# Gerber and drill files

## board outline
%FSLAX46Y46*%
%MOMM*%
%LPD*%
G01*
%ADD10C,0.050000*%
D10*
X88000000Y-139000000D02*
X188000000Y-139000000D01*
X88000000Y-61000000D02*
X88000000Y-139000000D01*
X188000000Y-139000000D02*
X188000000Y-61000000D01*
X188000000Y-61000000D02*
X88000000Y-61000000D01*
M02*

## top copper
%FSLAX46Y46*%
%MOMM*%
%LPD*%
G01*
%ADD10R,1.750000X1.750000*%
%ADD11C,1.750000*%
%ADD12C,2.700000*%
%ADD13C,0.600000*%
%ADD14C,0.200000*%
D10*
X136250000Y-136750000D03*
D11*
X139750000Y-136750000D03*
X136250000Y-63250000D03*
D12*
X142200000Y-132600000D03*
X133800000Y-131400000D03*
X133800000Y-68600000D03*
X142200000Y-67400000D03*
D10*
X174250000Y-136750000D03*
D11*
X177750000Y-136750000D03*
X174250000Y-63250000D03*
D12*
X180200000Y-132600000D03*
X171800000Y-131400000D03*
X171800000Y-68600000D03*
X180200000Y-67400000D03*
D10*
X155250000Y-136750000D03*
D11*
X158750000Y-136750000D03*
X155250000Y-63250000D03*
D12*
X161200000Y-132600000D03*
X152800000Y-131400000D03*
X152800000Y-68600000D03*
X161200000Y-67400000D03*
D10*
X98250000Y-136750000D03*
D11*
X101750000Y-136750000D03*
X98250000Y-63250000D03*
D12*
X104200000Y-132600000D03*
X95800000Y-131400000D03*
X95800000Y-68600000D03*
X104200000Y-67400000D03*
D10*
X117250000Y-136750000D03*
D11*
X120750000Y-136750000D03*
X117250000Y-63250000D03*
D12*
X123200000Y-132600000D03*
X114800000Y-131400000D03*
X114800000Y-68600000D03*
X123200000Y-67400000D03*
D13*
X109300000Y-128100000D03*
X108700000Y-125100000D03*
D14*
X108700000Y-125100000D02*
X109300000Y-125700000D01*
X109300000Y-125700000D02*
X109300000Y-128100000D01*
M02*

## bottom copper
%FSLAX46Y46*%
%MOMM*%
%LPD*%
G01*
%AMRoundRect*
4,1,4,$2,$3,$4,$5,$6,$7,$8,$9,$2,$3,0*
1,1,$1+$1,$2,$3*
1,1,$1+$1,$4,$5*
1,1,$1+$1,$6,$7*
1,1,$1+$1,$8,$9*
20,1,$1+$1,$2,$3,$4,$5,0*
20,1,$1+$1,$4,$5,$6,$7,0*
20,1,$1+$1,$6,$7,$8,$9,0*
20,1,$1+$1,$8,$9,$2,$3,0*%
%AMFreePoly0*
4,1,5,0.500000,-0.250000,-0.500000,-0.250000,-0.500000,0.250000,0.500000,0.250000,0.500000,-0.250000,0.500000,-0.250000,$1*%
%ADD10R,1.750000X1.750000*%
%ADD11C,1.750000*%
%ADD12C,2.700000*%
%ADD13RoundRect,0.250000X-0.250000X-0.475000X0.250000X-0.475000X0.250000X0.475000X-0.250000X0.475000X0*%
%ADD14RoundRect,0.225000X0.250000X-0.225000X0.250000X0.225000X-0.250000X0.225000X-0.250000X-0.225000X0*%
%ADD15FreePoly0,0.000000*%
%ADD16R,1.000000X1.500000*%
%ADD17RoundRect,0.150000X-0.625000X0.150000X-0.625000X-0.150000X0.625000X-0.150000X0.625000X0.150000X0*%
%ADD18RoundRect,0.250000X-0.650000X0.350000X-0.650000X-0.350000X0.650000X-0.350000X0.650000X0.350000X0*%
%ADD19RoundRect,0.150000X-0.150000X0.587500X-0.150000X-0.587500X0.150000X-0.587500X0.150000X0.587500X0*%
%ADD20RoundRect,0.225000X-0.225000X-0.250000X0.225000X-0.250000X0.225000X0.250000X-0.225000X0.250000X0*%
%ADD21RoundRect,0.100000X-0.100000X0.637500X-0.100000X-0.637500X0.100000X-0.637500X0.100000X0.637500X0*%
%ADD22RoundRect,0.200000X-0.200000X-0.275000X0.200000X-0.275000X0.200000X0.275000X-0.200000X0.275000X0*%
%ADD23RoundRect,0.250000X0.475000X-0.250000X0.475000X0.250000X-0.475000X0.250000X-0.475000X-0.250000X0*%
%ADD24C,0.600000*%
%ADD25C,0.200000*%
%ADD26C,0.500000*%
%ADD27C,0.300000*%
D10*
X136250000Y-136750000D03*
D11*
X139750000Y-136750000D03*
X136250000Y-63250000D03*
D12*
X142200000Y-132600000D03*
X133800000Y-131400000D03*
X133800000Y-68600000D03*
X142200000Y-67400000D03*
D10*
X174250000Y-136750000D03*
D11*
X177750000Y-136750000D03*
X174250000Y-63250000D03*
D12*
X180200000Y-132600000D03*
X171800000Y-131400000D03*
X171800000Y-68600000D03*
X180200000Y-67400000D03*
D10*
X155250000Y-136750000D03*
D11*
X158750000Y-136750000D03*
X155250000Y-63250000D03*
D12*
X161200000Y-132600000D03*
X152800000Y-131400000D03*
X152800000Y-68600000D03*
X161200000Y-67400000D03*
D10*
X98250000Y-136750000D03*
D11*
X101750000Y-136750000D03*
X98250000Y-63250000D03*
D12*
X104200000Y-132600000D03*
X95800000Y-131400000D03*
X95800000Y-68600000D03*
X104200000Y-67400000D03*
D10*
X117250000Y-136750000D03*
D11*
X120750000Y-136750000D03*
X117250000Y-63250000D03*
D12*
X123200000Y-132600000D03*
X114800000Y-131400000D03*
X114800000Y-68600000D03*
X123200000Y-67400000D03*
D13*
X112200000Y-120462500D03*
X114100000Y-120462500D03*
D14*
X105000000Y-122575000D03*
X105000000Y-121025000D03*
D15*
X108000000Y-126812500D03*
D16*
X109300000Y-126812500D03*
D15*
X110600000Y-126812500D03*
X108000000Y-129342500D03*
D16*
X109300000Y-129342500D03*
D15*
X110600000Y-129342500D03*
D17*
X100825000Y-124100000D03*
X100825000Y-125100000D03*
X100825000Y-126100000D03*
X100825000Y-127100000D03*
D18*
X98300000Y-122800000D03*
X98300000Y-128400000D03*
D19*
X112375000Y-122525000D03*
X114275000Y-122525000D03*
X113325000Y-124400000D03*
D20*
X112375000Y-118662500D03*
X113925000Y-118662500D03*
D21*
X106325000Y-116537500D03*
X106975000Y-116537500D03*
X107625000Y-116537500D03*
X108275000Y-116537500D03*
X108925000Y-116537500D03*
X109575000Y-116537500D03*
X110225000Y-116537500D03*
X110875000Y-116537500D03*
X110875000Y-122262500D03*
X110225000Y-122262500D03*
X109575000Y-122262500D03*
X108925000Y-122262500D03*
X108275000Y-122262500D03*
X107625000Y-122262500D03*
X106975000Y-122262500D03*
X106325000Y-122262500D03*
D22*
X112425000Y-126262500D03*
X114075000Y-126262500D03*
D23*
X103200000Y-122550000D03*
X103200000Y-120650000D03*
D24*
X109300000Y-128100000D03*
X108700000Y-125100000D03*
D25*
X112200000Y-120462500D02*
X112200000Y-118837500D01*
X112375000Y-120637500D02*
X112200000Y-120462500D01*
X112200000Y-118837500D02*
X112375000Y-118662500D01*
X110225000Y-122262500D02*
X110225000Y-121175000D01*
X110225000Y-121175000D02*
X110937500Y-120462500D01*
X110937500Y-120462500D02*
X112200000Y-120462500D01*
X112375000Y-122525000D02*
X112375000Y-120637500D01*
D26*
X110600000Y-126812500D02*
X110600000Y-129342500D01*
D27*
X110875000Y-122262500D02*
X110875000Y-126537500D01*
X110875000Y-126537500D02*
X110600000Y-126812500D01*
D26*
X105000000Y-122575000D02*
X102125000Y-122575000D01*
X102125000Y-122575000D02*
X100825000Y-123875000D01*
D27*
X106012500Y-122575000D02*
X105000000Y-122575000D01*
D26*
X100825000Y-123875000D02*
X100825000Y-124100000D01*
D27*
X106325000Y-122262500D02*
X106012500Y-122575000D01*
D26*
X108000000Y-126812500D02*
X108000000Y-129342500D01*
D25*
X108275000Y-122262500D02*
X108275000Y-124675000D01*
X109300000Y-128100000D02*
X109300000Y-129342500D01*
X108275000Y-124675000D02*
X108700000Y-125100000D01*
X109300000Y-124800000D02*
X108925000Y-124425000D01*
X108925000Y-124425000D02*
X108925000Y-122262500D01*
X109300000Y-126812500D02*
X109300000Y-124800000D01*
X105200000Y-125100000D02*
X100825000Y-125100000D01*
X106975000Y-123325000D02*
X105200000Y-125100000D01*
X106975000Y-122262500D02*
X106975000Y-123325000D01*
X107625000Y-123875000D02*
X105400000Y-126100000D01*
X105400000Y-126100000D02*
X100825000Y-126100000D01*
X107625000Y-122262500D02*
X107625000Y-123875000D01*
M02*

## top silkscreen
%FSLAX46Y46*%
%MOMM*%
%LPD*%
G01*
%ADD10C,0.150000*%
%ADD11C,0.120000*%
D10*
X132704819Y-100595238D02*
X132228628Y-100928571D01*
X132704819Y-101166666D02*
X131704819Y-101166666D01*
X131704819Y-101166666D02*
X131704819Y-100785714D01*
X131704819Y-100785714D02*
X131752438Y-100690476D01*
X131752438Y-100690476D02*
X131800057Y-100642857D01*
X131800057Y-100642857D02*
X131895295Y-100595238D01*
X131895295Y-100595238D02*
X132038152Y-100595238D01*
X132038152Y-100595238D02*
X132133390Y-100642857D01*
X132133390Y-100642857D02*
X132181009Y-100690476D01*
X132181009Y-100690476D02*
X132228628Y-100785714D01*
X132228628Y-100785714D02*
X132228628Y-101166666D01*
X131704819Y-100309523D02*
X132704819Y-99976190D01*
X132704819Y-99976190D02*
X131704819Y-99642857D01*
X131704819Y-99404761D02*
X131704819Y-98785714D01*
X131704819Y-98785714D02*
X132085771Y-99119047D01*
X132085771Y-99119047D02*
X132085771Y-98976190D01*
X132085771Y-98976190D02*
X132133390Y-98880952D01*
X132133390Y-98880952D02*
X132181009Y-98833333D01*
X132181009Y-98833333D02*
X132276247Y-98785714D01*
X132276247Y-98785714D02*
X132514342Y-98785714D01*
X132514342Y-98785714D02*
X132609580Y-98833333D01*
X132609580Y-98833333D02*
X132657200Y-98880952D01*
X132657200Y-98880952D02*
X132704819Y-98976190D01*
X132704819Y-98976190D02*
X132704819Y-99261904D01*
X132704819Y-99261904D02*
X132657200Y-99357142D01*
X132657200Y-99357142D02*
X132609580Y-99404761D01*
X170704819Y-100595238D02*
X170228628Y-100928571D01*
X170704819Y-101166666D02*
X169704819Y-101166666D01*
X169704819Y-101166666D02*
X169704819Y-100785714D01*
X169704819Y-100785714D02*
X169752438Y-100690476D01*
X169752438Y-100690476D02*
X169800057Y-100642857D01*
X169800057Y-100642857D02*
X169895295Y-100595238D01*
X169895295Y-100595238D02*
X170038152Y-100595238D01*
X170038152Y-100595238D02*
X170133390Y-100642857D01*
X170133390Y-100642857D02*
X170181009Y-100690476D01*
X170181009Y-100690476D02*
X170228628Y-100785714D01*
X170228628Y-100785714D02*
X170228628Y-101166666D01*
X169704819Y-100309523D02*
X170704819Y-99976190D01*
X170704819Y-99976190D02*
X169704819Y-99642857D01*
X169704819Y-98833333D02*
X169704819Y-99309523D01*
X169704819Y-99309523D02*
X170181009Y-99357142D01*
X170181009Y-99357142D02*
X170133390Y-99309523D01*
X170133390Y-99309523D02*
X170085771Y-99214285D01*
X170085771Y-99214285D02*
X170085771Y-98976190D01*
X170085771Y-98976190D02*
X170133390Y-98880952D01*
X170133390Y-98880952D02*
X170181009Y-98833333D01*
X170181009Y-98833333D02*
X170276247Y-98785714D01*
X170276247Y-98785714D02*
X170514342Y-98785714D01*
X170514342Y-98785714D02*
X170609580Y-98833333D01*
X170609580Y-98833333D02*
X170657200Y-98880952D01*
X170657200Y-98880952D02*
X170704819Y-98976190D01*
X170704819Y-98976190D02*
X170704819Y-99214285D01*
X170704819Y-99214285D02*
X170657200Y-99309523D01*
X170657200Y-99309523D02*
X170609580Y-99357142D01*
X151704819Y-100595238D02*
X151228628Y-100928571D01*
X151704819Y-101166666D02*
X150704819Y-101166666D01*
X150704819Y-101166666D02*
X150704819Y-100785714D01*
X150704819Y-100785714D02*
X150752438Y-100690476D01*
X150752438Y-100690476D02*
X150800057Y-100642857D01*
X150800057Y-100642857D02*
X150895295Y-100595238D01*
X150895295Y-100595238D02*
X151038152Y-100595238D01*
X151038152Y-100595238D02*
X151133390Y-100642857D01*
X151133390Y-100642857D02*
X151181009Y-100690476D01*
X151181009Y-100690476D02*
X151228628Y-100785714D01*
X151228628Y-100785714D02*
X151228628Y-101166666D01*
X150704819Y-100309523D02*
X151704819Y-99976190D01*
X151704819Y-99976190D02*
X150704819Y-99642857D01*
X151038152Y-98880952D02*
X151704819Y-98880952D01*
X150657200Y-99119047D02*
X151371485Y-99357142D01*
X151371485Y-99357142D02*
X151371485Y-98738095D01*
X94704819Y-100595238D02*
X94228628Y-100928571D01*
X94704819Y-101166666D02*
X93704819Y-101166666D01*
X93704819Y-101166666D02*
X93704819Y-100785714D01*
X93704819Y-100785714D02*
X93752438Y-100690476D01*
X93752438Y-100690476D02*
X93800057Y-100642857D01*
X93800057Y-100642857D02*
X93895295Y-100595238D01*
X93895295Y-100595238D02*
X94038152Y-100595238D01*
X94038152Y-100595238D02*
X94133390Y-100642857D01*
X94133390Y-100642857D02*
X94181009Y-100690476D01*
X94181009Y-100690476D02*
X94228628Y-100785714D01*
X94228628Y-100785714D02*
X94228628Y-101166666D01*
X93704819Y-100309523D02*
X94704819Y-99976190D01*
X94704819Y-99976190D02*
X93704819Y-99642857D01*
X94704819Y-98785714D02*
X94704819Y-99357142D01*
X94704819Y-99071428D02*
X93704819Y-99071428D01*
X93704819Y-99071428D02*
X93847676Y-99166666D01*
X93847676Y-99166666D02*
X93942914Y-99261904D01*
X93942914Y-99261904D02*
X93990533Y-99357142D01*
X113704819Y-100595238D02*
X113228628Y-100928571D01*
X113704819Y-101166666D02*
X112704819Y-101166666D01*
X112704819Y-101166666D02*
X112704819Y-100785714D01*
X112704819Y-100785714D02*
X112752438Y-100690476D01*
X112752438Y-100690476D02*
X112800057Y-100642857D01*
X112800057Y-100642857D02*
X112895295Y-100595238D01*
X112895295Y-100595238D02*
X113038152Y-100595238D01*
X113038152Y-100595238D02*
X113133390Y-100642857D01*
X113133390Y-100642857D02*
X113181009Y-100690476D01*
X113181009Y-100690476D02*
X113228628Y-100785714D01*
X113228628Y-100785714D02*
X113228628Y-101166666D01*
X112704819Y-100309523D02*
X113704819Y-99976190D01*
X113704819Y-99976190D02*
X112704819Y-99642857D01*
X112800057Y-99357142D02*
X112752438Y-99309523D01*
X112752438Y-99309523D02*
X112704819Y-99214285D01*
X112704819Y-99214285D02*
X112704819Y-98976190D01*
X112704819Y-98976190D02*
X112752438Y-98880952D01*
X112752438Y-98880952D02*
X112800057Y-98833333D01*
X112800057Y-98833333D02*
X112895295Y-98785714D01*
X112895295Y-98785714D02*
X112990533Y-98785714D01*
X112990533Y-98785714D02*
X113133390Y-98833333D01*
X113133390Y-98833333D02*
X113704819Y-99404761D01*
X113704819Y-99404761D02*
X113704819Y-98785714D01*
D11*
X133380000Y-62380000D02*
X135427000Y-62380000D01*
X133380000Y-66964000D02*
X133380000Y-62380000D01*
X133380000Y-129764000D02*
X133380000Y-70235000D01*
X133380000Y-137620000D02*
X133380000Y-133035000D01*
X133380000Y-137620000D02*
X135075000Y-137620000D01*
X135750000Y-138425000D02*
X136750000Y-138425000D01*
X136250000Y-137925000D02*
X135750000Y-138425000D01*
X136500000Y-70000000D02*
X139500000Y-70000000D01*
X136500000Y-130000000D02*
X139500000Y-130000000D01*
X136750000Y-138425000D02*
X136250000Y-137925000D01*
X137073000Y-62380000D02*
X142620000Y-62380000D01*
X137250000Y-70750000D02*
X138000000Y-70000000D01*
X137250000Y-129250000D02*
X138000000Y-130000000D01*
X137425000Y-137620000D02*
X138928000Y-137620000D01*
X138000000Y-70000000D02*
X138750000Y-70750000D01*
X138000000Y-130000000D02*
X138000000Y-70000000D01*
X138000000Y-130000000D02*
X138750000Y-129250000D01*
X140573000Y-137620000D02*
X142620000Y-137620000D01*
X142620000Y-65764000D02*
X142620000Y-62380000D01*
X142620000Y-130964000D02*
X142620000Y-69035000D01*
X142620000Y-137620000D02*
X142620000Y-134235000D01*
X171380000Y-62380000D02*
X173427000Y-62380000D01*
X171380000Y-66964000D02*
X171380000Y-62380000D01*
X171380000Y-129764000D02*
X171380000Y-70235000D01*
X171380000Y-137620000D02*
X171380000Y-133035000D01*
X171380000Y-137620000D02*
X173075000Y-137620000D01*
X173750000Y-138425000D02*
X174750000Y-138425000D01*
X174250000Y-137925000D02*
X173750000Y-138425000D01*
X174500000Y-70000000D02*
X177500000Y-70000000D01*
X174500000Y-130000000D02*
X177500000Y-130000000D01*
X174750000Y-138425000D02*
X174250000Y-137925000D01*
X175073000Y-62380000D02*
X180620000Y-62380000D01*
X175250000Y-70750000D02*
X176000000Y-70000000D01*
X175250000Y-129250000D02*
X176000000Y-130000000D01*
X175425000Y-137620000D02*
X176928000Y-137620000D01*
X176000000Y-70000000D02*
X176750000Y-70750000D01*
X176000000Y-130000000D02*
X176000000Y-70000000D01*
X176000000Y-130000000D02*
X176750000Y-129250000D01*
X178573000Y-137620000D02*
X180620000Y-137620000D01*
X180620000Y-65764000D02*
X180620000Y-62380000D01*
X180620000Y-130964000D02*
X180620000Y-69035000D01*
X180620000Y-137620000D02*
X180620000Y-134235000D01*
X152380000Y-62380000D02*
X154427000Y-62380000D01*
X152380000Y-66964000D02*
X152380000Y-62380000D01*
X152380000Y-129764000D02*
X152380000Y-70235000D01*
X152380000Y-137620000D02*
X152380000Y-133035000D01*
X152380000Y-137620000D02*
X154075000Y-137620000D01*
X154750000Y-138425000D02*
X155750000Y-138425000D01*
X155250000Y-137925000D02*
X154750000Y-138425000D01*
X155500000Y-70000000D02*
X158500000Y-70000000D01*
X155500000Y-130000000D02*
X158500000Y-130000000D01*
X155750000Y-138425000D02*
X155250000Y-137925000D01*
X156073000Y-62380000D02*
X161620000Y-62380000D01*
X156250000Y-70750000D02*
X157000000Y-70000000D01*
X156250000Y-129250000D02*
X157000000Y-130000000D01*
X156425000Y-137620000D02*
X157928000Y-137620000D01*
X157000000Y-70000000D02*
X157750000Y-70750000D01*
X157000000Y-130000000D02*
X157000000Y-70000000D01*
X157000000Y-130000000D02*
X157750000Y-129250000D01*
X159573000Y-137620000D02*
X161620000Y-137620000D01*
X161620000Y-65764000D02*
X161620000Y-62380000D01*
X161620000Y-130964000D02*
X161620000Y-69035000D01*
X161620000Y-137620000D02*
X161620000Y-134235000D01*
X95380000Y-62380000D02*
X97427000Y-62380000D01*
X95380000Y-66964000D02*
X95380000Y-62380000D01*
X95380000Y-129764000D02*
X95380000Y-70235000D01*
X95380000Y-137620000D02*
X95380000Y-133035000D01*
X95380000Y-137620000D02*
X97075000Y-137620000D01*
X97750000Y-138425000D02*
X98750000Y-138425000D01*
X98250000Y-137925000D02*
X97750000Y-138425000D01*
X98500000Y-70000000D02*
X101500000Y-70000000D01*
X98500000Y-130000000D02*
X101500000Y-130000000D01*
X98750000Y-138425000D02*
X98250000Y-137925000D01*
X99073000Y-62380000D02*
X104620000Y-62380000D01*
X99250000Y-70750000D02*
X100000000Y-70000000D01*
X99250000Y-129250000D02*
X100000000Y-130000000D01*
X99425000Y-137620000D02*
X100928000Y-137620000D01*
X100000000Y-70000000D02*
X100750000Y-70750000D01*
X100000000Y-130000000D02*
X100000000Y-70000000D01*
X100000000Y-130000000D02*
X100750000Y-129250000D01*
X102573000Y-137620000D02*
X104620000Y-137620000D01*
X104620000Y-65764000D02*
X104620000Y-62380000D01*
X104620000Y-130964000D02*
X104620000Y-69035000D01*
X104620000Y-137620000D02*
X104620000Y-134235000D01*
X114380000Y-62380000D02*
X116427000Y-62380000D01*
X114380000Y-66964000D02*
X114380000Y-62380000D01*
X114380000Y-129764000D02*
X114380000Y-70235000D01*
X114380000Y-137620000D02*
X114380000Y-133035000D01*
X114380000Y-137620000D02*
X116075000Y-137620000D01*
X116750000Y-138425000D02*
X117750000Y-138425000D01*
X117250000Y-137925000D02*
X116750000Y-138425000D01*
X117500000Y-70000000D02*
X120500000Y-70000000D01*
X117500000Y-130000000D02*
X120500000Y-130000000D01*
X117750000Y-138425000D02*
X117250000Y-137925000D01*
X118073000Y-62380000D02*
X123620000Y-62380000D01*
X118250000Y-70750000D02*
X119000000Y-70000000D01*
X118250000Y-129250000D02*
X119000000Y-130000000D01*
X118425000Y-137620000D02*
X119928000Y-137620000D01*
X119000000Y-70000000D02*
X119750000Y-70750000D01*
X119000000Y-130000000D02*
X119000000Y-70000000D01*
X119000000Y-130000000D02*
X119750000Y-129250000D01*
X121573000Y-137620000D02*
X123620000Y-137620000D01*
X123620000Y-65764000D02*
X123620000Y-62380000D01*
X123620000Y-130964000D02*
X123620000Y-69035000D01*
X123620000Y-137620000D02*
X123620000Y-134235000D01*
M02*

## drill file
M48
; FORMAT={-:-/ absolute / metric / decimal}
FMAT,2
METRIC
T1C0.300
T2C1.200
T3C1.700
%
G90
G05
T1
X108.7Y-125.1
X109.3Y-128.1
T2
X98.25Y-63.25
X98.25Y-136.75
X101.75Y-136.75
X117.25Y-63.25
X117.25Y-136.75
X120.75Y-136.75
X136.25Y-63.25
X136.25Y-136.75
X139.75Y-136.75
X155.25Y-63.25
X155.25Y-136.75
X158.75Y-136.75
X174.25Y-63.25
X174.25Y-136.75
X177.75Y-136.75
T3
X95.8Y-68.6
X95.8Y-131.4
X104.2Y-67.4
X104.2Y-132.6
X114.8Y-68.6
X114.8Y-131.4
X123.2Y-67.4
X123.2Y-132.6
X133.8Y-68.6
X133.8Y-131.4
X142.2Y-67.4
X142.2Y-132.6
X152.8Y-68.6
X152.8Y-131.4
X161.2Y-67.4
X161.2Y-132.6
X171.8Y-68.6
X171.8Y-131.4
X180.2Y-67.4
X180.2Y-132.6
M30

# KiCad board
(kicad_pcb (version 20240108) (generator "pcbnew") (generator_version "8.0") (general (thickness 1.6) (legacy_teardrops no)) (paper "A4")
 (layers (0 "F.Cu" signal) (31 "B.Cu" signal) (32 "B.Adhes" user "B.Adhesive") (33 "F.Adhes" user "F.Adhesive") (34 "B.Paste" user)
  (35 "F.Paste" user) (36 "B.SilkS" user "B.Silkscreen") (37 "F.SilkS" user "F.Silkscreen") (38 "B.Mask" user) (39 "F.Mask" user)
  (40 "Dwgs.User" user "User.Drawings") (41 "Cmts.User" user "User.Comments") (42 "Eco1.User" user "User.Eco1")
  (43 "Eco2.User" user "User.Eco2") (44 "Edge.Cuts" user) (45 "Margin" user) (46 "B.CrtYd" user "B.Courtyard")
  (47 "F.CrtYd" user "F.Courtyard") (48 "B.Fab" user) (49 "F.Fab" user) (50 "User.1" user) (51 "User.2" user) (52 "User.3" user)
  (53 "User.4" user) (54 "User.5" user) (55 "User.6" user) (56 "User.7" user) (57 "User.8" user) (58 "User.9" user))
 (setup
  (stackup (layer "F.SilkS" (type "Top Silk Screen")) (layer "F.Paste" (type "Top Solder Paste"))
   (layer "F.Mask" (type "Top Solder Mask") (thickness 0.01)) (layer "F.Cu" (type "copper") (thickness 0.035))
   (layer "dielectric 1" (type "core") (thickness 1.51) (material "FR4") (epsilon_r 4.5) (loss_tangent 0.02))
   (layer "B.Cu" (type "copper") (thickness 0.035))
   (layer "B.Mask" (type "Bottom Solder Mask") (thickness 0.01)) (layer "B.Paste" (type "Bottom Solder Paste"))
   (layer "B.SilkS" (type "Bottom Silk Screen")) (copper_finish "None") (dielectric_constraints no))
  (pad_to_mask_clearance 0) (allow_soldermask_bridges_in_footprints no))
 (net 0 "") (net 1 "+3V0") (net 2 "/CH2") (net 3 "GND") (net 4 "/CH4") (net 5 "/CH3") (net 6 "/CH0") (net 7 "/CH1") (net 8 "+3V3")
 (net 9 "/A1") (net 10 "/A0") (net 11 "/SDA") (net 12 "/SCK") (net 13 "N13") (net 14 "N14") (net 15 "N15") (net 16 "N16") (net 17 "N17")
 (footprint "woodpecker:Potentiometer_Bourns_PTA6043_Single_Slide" (layer "F.Cu") (at 138 100 90)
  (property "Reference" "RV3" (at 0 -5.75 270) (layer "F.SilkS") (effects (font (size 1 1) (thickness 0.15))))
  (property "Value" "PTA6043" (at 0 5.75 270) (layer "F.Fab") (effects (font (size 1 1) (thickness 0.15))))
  (fp_line (start 37.62 -4.62) (end 37.62 -2.573) (stroke (width 0.12) (type solid)) (layer "F.SilkS"))
  (fp_line (start 33.036 -4.62) (end 37.62 -4.62) (stroke (width 0.12) (type solid)) (layer "F.SilkS"))
  (fp_line (start -29.764 -4.62) (end 29.765 -4.62) (stroke (width 0.12) (type solid)) (layer "F.SilkS"))
  (fp_line (start -37.62 -4.62) (end -33.035 -4.62) (stroke (width 0.12) (type solid)) (layer "F.SilkS"))
  (fp_line (start -37.62 -4.62) (end -37.62 -2.925) (stroke (width 0.12) (type solid)) (layer "F.SilkS"))
  (fp_line (start -38.425 -2.25) (end -38.425 -1.25) (stroke (width 0.12) (type solid)) (layer "F.SilkS"))
  (fp_line (start -37.925 -1.75) (end -38.425 -2.25) (stroke (width 0.12) (type solid)) (layer "F.SilkS"))
  (fp_line (start 30 -1.5) (end 30 1.5) (stroke (width 0.12) (type solid)) (layer "F.SilkS"))
  (fp_line (start -30 -1.5) (end -30 1.5) (stroke (width 0.12) (type solid)) (layer "F.SilkS"))
  (fp_line (start -38.425 -1.25) (end -37.925 -1.75) (stroke (width 0.12) (type solid)) (layer "F.SilkS"))
  (fp_line (start 37.62 -0.927) (end 37.62 4.62) (stroke (width 0.12) (type solid)) (layer "F.SilkS"))
  (fp_line (start 29.25 -0.75) (end 30 0) (stroke (width 0.12) (type solid)) (layer "F.SilkS"))
  (fp_line (start -29.25 -0.75) (end -30 0) (stroke (width 0.12) (type solid)) (layer "F.SilkS"))
  (fp_line (start -37.62 -0.575) (end -37.62 0.928) (stroke (width 0.12) (type solid)) (layer "F.SilkS"))
  (fp_line (start 30 0) (end 29.25 0.75) (stroke (width 0.12) (type solid)) (layer "F.SilkS"))
  (fp_line (start -30 0) (end 30 0) (stroke (width 0.12) (type solid)) (layer "F.SilkS"))
  (fp_line (start -30 0) (end -29.25 0.75) (stroke (width 0.12) (type solid)) (layer "F.SilkS"))
  (fp_line (start -37.62 2.573) (end -37.62 4.62) (stroke (width 0.12) (type solid)) (layer "F.SilkS"))
  (fp_line (start 34.236 4.62) (end 37.62 4.62) (stroke (width 0.12) (type solid)) (layer "F.SilkS"))
  (fp_line (start -30.964 4.62) (end 30.965 4.62) (stroke (width 0.12) (type solid)) (layer "F.SilkS"))
  (fp_line (start -37.62 4.62) (end -34.235 4.62) (stroke (width 0.12) (type solid)) (layer "F.SilkS"))
  (pad "1" thru_hole rect (at -36.75 -1.75 90) (size 1.75 1.75) (drill 1.2) (layers "*.Cu" "*.Mask") (remove_unused_layers no)
   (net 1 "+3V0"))
  (pad "2" thru_hole circle (at -36.75 1.75 90) (size 1.75 1.75) (drill 1.2) (layers "*.Cu" "*.Mask") (remove_unused_layers no)
   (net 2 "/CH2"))
  (pad "3" thru_hole circle (at 36.75 -1.75 90) (size 1.75 1.75) (drill 1.2) (layers "*.Cu" "*.Mask") (remove_unused_layers no)
   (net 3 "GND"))
  (pad "MP" thru_hole circle (at -32.6 4.2 90) (size 2.7 2.7) (drill 1.7) (layers "*.Cu" "*.Mask") (remove_unused_layers no))
  (pad "MP" thru_hole circle (at -31.4 -4.2 90) (size 2.7 2.7) (drill 1.7) (layers "*.Cu" "*.Mask") (remove_unused_layers no))
  (pad "MP" thru_hole circle (at 31.4 -4.2 90) (size 2.7 2.7) (drill 1.7) (layers "*.Cu" "*.Mask") (remove_unused_layers no))
  (pad "MP" thru_hole circle (at 32.6 4.2 90) (size 2.7 2.7) (drill 1.7) (layers "*.Cu" "*.Mask") (remove_unused_layers no)))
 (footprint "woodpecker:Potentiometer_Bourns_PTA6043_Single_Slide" (layer "F.Cu") (at 176 100 90)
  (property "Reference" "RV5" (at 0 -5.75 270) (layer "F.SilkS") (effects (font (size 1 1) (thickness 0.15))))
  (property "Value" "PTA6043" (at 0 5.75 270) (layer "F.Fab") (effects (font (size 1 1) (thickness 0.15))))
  (fp_line (start 37.62 -4.62) (end 37.62 -2.573) (stroke (width 0.12) (type solid)) (layer "F.SilkS"))
  (fp_line (start 33.036 -4.62) (end 37.62 -4.62) (stroke (width 0.12) (type solid)) (layer "F.SilkS"))
  (fp_line (start -29.764 -4.62) (end 29.765 -4.62) (stroke (width 0.12) (type solid)) (layer "F.SilkS"))
  (fp_line (start -37.62 -4.62) (end -33.035 -4.62) (stroke (width 0.12) (type solid)) (layer "F.SilkS"))
  (fp_line (start -37.62 -4.62) (end -37.62 -2.925) (stroke (width 0.12) (type solid)) (layer "F.SilkS"))
  (fp_line (start -38.425 -2.25) (end -38.425 -1.25) (stroke (width 0.12) (type solid)) (layer "F.SilkS"))
  (fp_line (start -37.925 -1.75) (end -38.425 -2.25) (stroke (width 0.12) (type solid)) (layer "F.SilkS"))
  (fp_line (start 30 -1.5) (end 30 1.5) (stroke (width 0.12) (type solid)) (layer "F.SilkS"))
  (fp_line (start -30 -1.5) (end -30 1.5) (stroke (width 0.12) (type solid)) (layer "F.SilkS"))
  (fp_line (start -38.425 -1.25) (end -37.925 -1.75) (stroke (width 0.12) (type solid)) (layer "F.SilkS"))
  (fp_line (start 37.62 -0.927) (end 37.62 4.62) (stroke (width 0.12) (type solid)) (layer "F.SilkS"))
  (fp_line (start 29.25 -0.75) (end 30 0) (stroke (width 0.12) (type solid)) (layer "F.SilkS"))
  (fp_line (start -29.25 -0.75) (end -30 0) (stroke (width 0.12) (type solid)) (layer "F.SilkS"))
  (fp_line (start -37.62 -0.575) (end -37.62 0.928) (stroke (width 0.12) (type solid)) (layer "F.SilkS"))
  (fp_line (start 30 0) (end 29.25 0.75) (stroke (width 0.12) (type solid)) (layer "F.SilkS"))
  (fp_line (start -30 0) (end 30 0) (stroke (width 0.12) (type solid)) (layer "F.SilkS"))
  (fp_line (start -30 0) (end -29.25 0.75) (stroke (width 0.12) (type solid)) (layer "F.SilkS"))
  (fp_line (start -37.62 2.573) (end -37.62 4.62) (stroke (width 0.12) (type solid)) (layer "F.SilkS"))
  (fp_line (start 34.236 4.62) (end 37.62 4.62) (stroke (width 0.12) (type solid)) (layer "F.SilkS"))
  (fp_line (start -30.964 4.62) (end 30.965 4.62) (stroke (width 0.12) (type solid)) (layer "F.SilkS"))
  (fp_line (start -37.62 4.62) (end -34.235 4.62) (stroke (width 0.12) (type solid)) (layer "F.SilkS"))
  (pad "1" thru_hole rect (at -36.75 -1.75 90) (size 1.75 1.75) (drill 1.2) (layers "*.Cu" "*.Mask") (remove_unused_layers no)
   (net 1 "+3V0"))
  (pad "2" thru_hole circle (at -36.75 1.75 90) (size 1.75 1.75) (drill 1.2) (layers "*.Cu" "*.Mask") (remove_unused_layers no)
   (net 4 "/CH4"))
  (pad "3" thru_hole circle (at 36.75 -1.75 90) (size 1.75 1.75) (drill 1.2) (layers "*.Cu" "*.Mask") (remove_unused_layers no)
   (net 3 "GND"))
  (pad "MP" thru_hole circle (at -32.6 4.2 90) (size 2.7 2.7) (drill 1.7) (layers "*.Cu" "*.Mask") (remove_unused_layers no))
  (pad "MP" thru_hole circle (at -31.4 -4.2 90) (size 2.7 2.7) (drill 1.7) (layers "*.Cu" "*.Mask") (remove_unused_layers no))
  (pad "MP" thru_hole circle (at 31.4 -4.2 90) (size 2.7 2.7) (drill 1.7) (layers "*.Cu" "*.Mask") (remove_unused_layers no))
  (pad "MP" thru_hole circle (at 32.6 4.2 90) (size 2.7 2.7) (drill 1.7) (layers "*.Cu" "*.Mask") (remove_unused_layers no)))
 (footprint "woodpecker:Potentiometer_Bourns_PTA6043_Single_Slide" (layer "F.Cu") (at 157 100 90)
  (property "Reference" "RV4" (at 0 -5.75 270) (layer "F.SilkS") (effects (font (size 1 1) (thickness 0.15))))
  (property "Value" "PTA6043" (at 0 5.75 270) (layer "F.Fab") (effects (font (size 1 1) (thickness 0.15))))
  (fp_line (start 37.62 -4.62) (end 37.62 -2.573) (stroke (width 0.12) (type solid)) (layer "F.SilkS"))
  (fp_line (start 33.036 -4.62) (end 37.62 -4.62) (stroke (width 0.12) (type solid)) (layer "F.SilkS"))
  (fp_line (start -29.764 -4.62) (end 29.765 -4.62) (stroke (width 0.12) (type solid)) (layer "F.SilkS"))
  (fp_line (start -37.62 -4.62) (end -33.035 -4.62) (stroke (width 0.12) (type solid)) (layer "F.SilkS"))
  (fp_line (start -37.62 -4.62) (end -37.62 -2.925) (stroke (width 0.12) (type solid)) (layer "F.SilkS"))
  (fp_line (start -38.425 -2.25) (end -38.425 -1.25) (stroke (width 0.12) (type solid)) (layer "F.SilkS"))
  (fp_line (start -37.925 -1.75) (end -38.425 -2.25) (stroke (width 0.12) (type solid)) (layer "F.SilkS"))
  (fp_line (start 30 -1.5) (end 30 1.5) (stroke (width 0.12) (type solid)) (layer "F.SilkS"))
  (fp_line (start -30 -1.5) (end -30 1.5) (stroke (width 0.12) (type solid)) (layer "F.SilkS"))
  (fp_line (start -38.425 -1.25) (end -37.925 -1.75) (stroke (width 0.12) (type solid)) (layer "F.SilkS"))
  (fp_line (start 37.62 -0.927) (end 37.62 4.62) (stroke (width 0.12) (type solid)) (layer "F.SilkS"))
  (fp_line (start 29.25 -0.75) (end 30 0) (stroke (width 0.12) (type solid)) (layer "F.SilkS"))
  (fp_line (start -29.25 -0.75) (end -30 0) (stroke (width 0.12) (type solid)) (layer "F.SilkS"))
  (fp_line (start -37.62 -0.575) (end -37.62 0.928) (stroke (width 0.12) (type solid)) (layer "F.SilkS"))
  (fp_line (start 30 0) (end 29.25 0.75) (stroke (width 0.12) (type solid)) (layer "F.SilkS"))
  (fp_line (start -30 0) (end 30 0) (stroke (width 0.12) (type solid)) (layer "F.SilkS"))
  (fp_line (start -30 0) (end -29.25 0.75) (stroke (width 0.12) (type solid)) (layer "F.SilkS"))
  (fp_line (start -37.62 2.573) (end -37.62 4.62) (stroke (width 0.12) (type solid)) (layer "F.SilkS"))
  (fp_line (start 34.236 4.62) (end 37.62 4.62) (stroke (width 0.12) (type solid)) (layer "F.SilkS"))
  (fp_line (start -30.964 4.62) (end 30.965 4.62) (stroke (width 0.12) (type solid)) (layer "F.SilkS"))
  (fp_line (start -37.62 4.62) (end -34.235 4.62) (stroke (width 0.12) (type solid)) (layer "F.SilkS"))
  (pad "1" thru_hole rect (at -36.75 -1.75 90) (size 1.75 1.75) (drill 1.2) (layers "*.Cu" "*.Mask") (remove_unused_layers no)
   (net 1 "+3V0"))
  (pad "2" thru_hole circle (at -36.75 1.75 90) (size 1.75 1.75) (drill 1.2) (layers "*.Cu" "*.Mask") (remove_unused_layers no)
   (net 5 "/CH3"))
  (pad "3" thru_hole circle (at 36.75 -1.75 90) (size 1.75 1.75) (drill 1.2) (layers "*.Cu" "*.Mask") (remove_unused_layers no)
   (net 3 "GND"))
  (pad "MP" thru_hole circle (at -32.6 4.2 90) (size 2.7 2.7) (drill 1.7) (layers "*.Cu" "*.Mask") (remove_unused_layers no))
  (pad "MP" thru_hole circle (at -31.4 -4.2 90) (size 2.7 2.7) (drill 1.7) (layers "*.Cu" "*.Mask") (remove_unused_layers no))
  (pad "MP" thru_hole circle (at 31.4 -4.2 90) (size 2.7 2.7) (drill 1.7) (layers "*.Cu" "*.Mask") (remove_unused_layers no))
  (pad "MP" thru_hole circle (at 32.6 4.2 90) (size 2.7 2.7) (drill 1.7) (layers "*.Cu" "*.Mask") (remove_unused_layers no)))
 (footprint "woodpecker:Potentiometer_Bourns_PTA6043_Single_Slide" (layer "F.Cu") (at 100 100 90)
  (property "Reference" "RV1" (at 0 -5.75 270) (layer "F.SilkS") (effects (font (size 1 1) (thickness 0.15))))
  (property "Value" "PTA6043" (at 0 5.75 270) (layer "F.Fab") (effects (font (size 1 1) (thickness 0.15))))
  (fp_line (start 37.62 -4.62) (end 37.62 -2.573) (stroke (width 0.12) (type solid)) (layer "F.SilkS"))
  (fp_line (start 33.036 -4.62) (end 37.62 -4.62) (stroke (width 0.12) (type solid)) (layer "F.SilkS"))
  (fp_line (start -29.764 -4.62) (end 29.765 -4.62) (stroke (width 0.12) (type solid)) (layer "F.SilkS"))
  (fp_line (start -37.62 -4.62) (end -33.035 -4.62) (stroke (width 0.12) (type solid)) (layer "F.SilkS"))
  (fp_line (start -37.62 -4.62) (end -37.62 -2.925) (stroke (width 0.12) (type solid)) (layer "F.SilkS"))
  (fp_line (start -38.425 -2.25) (end -38.425 -1.25) (stroke (width 0.12) (type solid)) (layer "F.SilkS"))
  (fp_line (start -37.925 -1.75) (end -38.425 -2.25) (stroke (width 0.12) (type solid)) (layer "F.SilkS"))
  (fp_line (start 30 -1.5) (end 30 1.5) (stroke (width 0.12) (type solid)) (layer "F.SilkS"))
  (fp_line (start -30 -1.5) (end -30 1.5) (stroke (width 0.12) (type solid)) (layer "F.SilkS"))
  (fp_line (start -38.425 -1.25) (end -37.925 -1.75) (stroke (width 0.12) (type solid)) (layer "F.SilkS"))
  (fp_line (start 37.62 -0.927) (end 37.62 4.62) (stroke (width 0.12) (type solid)) (layer "F.SilkS"))
  (fp_line (start 29.25 -0.75) (end 30 0) (stroke (width 0.12) (type solid)) (layer "F.SilkS"))
  (fp_line (start -29.25 -0.75) (end -30 0) (stroke (width 0.12) (type solid)) (layer "F.SilkS"))
  (fp_line (start -37.62 -0.575) (end -37.62 0.928) (stroke (width 0.12) (type solid)) (layer "F.SilkS"))
  (fp_line (start 30 0) (end 29.25 0.75) (stroke (width 0.12) (type solid)) (layer "F.SilkS"))
  (fp_line (start -30 0) (end 30 0) (stroke (width 0.12) (type solid)) (layer "F.SilkS"))
  (fp_line (start -30 0) (end -29.25 0.75) (stroke (width 0.12) (type solid)) (layer "F.SilkS"))
  (fp_line (start -37.62 2.573) (end -37.62 4.62) (stroke (width 0.12) (type solid)) (layer "F.SilkS"))
  (fp_line (start 34.236 4.62) (end 37.62 4.62) (stroke (width 0.12) (type solid)) (layer "F.SilkS"))
  (fp_line (start -30.964 4.62) (end 30.965 4.62) (stroke (width 0.12) (type solid)) (layer "F.SilkS"))
  (fp_line (start -37.62 4.62) (end -34.235 4.62) (stroke (width 0.12) (type solid)) (layer "F.SilkS"))
  (pad "1" thru_hole rect (at -36.75 -1.75 90) (size 1.75 1.75) (drill 1.2) (layers "*.Cu" "*.Mask") (remove_unused_layers no)
   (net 1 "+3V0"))
  (pad "2" thru_hole circle (at -36.75 1.75 90) (size 1.75 1.75) (drill 1.2) (layers "*.Cu" "*.Mask") (remove_unused_layers no)
   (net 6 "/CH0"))
  (pad "3" thru_hole circle (at 36.75 -1.75 90) (size 1.75 1.75) (drill 1.2) (layers "*.Cu" "*.Mask") (remove_unused_layers no)
   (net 3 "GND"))
  (pad "MP" thru_hole circle (at -32.6 4.2 90) (size 2.7 2.7) (drill 1.7) (layers "*.Cu" "*.Mask") (remove_unused_layers no))
  (pad "MP" thru_hole circle (at -31.4 -4.2 90) (size 2.7 2.7) (drill 1.7) (layers "*.Cu" "*.Mask") (remove_unused_layers no))
  (pad "MP" thru_hole circle (at 31.4 -4.2 90) (size 2.7 2.7) (drill 1.7) (layers "*.Cu" "*.Mask") (remove_unused_layers no))
  (pad "MP" thru_hole circle (at 32.6 4.2 90) (size 2.7 2.7) (drill 1.7) (layers "*.Cu" "*.Mask") (remove_unused_layers no)))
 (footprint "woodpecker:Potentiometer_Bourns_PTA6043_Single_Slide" (layer "F.Cu") (at 119 100 90)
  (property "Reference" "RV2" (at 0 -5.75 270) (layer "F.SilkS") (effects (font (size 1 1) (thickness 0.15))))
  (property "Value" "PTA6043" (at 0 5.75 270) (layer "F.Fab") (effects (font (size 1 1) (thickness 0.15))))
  (fp_line (start 37.62 -4.62) (end 37.62 -2.573) (stroke (width 0.12) (type solid)) (layer "F.SilkS"))
  (fp_line (start 33.036 -4.62) (end 37.62 -4.62) (stroke (width 0.12) (type solid)) (layer "F.SilkS"))
  (fp_line (start -29.764 -4.62) (end 29.765 -4.62) (stroke (width 0.12) (type solid)) (layer "F.SilkS"))
  (fp_line (start -37.62 -4.62) (end -33.035 -4.62) (stroke (width 0.12) (type solid)) (layer "F.SilkS"))
  (fp_line (start -37.62 -4.62) (end -37.62 -2.925) (stroke (width 0.12) (type solid)) (layer "F.SilkS"))
  (fp_line (start -38.425 -2.25) (end -38.425 -1.25) (stroke (width 0.12) (type solid)) (layer "F.SilkS"))
  (fp_line (start -37.925 -1.75) (end -38.425 -2.25) (stroke (width 0.12) (type solid)) (layer "F.SilkS"))
  (fp_line (start 30 -1.5) (end 30 1.5) (stroke (width 0.12) (type solid)) (layer "F.SilkS"))
  (fp_line (start -30 -1.5) (end -30 1.5) (stroke (width 0.12) (type solid)) (layer "F.SilkS"))
  (fp_line (start -38.425 -1.25) (end -37.925 -1.75) (stroke (width 0.12) (type solid)) (layer "F.SilkS"))
  (fp_line (start 37.62 -0.927) (end 37.62 4.62) (stroke (width 0.12) (type solid)) (layer "F.SilkS"))
  (fp_line (start 29.25 -0.75) (end 30 0) (stroke (width 0.12) (type solid)) (layer "F.SilkS"))
  (fp_line (start -29.25 -0.75) (end -30 0) (stroke (width 0.12) (type solid)) (layer "F.SilkS"))
  (fp_line (start -37.62 -0.575) (end -37.62 0.928) (stroke (width 0.12) (type solid)) (layer "F.SilkS"))
  (fp_line (start 30 0) (end 29.25 0.75) (stroke (width 0.12) (type solid)) (layer "F.SilkS"))
  (fp_line (start -30 0) (end 30 0) (stroke (width 0.12) (type solid)) (layer "F.SilkS"))
  (fp_line (start -30 0) (end -29.25 0.75) (stroke (width 0.12) (type solid)) (layer "F.SilkS"))
  (fp_line (start -37.62 2.573) (end -37.62 4.62) (stroke (width 0.12) (type solid)) (layer "F.SilkS"))
  (fp_line (start 34.236 4.62) (end 37.62 4.62) (stroke (width 0.12) (type solid)) (layer "F.SilkS"))
  (fp_line (start -30.964 4.62) (end 30.965 4.62) (stroke (width 0.12) (type solid)) (layer "F.SilkS"))
  (fp_line (start -37.62 4.62) (end -34.235 4.62) (stroke (width 0.12) (type solid)) (layer "F.SilkS"))
  (pad "1" thru_hole rect (at -36.75 -1.75 90) (size 1.75 1.75) (drill 1.2) (layers "*.Cu" "*.Mask") (remove_unused_layers no)
   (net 1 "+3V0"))
  (pad "2" thru_hole circle (at -36.75 1.75 90) (size 1.75 1.75) (drill 1.2) (layers "*.Cu" "*.Mask") (remove_unused_layers no)
   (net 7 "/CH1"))
  (pad "3" thru_hole circle (at 36.75 -1.75 90) (size 1.75 1.75) (drill 1.2) (layers "*.Cu" "*.Mask") (remove_unused_layers no)
   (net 3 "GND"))
  (pad "MP" thru_hole circle (at -32.6 4.2 90) (size 2.7 2.7) (drill 1.7) (layers "*.Cu" "*.Mask") (remove_unused_layers no))
  (pad "MP" thru_hole circle (at -31.4 -4.2 90) (size 2.7 2.7) (drill 1.7) (layers "*.Cu" "*.Mask") (remove_unused_layers no))
  (pad "MP" thru_hole circle (at 31.4 -4.2 90) (size 2.7 2.7) (drill 1.7) (layers "*.Cu" "*.Mask") (remove_unused_layers no))
  (pad "MP" thru_hole circle (at 32.6 4.2 90) (size 2.7 2.7) (drill 1.7) (layers "*.Cu" "*.Mask") (remove_unused_layers no)))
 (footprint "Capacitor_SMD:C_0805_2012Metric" (layer "B.Cu") (at 113.15 120.4625)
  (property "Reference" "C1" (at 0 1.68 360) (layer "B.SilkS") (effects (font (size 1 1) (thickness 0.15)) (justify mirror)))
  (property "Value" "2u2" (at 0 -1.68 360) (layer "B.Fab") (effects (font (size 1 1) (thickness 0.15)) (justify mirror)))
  (pad "1" smd roundrect (at -0.95 0) (size 1 1.45) (layers "B.Cu" "B.Paste" "B.Mask") (roundrect_rratio 0.25) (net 1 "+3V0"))
  (pad "2" smd roundrect (at 0.95 0) (size 1 1.45) (layers "B.Cu" "B.Paste" "B.Mask") (roundrect_rratio 0.25) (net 3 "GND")))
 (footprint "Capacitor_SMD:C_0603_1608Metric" (layer "B.Cu") (at 105 121.8 90)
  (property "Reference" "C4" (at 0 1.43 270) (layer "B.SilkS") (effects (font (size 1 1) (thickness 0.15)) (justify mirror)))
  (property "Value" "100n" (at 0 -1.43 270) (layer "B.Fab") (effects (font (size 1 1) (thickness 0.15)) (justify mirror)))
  (pad "1" smd roundrect (at -0.775 0 90) (size 0.9 0.95) (layers "B.Cu" "B.Paste" "B.Mask") (roundrect_rratio 0.25) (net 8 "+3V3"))
  (pad "2" smd roundrect (at 0.775 0 90) (size 0.9 0.95) (layers "B.Cu" "B.Paste" "B.Mask") (roundrect_rratio 0.25) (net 3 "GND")))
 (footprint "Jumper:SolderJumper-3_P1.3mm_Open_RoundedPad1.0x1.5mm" (layer "B.Cu") (at 109.3 126.8125)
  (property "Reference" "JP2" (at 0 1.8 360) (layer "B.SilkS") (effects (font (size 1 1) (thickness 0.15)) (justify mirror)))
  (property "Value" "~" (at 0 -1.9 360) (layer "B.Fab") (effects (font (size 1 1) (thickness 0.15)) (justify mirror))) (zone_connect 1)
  (pad "1" smd custom (at -1.3 0) (size 1 0.5) (layers "B.Cu" "B.Mask") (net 8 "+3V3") (zone_connect 2) (thermal_bridge_angle 45)
   (options (clearance outline) (anchor rect)) (primitives))
  (pad "2" smd rect (at 0 0) (size 1 1.5) (layers "B.Cu" "B.Mask") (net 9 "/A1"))
  (pad "3" smd custom (at 1.3 0) (size 1 0.5) (layers "B.Cu" "B.Mask") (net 3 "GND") (zone_connect 2) (thermal_bridge_angle 45)
   (options (clearance outline) (anchor rect)) (primitives)))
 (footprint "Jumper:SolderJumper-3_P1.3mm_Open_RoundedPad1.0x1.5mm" (layer "B.Cu") (at 109.3 129.3425)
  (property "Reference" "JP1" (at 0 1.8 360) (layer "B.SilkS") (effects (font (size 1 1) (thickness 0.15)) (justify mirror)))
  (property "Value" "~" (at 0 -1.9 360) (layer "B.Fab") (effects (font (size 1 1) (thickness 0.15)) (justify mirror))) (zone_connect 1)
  (pad "1" smd custom (at -1.3 0) (size 1 0.5) (layers "B.Cu" "B.Mask") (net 8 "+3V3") (zone_connect 2) (thermal_bridge_angle 45)
   (options (clearance outline) (anchor rect)) (primitives))
  (pad "2" smd rect (at 0 0) (size 1 1.5) (layers "B.Cu" "B.Mask") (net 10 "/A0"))
  (pad "3" smd custom (at 1.3 0) (size 1 0.5) (layers "B.Cu" "B.Mask") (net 3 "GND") (zone_connect 2) (thermal_bridge_angle 45)
   (options (clearance outline) (anchor rect)) (primitives)))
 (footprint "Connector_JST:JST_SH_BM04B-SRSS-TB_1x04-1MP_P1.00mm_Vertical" (layer "B.Cu") (at 99.5 125.6 -90)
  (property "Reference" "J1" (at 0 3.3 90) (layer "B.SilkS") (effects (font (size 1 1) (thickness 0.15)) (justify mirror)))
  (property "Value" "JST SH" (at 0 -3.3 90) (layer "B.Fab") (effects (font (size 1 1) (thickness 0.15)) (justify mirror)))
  (pad "1" smd roundrect (at -1.5 -1.325 270) (size 0.6 1.55) (layers "B.Cu" "B.Paste" "B.Mask") (roundrect_rratio 0.25) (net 8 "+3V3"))
  (pad "2" smd roundrect (at -0.5 -1.325 270) (size 0.6 1.55) (layers "B.Cu" "B.Paste" "B.Mask") (roundrect_rratio 0.25) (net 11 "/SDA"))
  (pad "3" smd roundrect (at 0.5 -1.325 270) (size 0.6 1.55) (layers "B.Cu" "B.Paste" "B.Mask") (roundrect_rratio 0.25) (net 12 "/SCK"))
  (pad "4" smd roundrect (at 1.5 -1.325 270) (size 0.6 1.55) (layers "B.Cu" "B.Paste" "B.Mask") (roundrect_rratio 0.25) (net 3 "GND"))
  (pad "MP" smd roundrect (at -2.8 1.2 270) (size 1.2 1.8) (layers "B.Cu" "B.Paste" "B.Mask") (roundrect_rratio 0.208333))
  (pad "MP" smd roundrect (at 2.8 1.2 270) (size 1.2 1.8) (layers "B.Cu" "B.Paste" "B.Mask") (roundrect_rratio 0.208333)))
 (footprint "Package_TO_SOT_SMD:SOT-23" (layer "B.Cu") (at 113.325 123.4625 -90)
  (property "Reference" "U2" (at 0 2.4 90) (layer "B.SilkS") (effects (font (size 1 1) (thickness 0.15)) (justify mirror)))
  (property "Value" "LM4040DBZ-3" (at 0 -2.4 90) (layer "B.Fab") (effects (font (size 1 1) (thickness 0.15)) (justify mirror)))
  (pad "1" smd roundrect (at -0.9375 0.95 270) (size 1.475 0.6) (layers "B.Cu" "B.Paste" "B.Mask") (roundrect_rratio 0.25) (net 1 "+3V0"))
  (pad "2" smd roundrect (at -0.9375 -0.95 270) (size 1.475 0.6) (layers "B.Cu" "B.Paste" "B.Mask") (roundrect_rratio 0.25) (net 3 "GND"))
  (pad "3" smd roundrect (at 0.9375 0 270) (size 1.475 0.6) (layers "B.Cu" "B.Paste" "B.Mask") (roundrect_rratio 0.25) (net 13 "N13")))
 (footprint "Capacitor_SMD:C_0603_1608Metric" (layer "B.Cu") (at 113.15 118.6625)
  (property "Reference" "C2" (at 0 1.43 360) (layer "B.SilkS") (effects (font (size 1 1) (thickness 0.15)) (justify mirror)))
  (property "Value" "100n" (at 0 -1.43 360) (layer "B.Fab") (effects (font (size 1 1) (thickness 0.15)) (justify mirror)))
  (pad "1" smd roundrect (at -0.775 0) (size 0.9 0.95) (layers "B.Cu" "B.Paste" "B.Mask") (roundrect_rratio 0.25) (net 1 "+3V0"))
  (pad "2" smd roundrect (at 0.775 0) (size 0.9 0.95) (layers "B.Cu" "B.Paste" "B.Mask") (roundrect_rratio 0.25) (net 3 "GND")))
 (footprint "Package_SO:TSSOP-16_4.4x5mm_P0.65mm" (layer "B.Cu") (at 108.6 119.4 -90)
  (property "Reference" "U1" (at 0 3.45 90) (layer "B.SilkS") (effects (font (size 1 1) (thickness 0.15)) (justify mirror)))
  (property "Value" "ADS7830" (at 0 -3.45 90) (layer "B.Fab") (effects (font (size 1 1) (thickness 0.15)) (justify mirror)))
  (pad "1" smd roundrect (at -2.8625 2.275 270) (size 1.475 0.4) (layers "B.Cu" "B.Paste" "B.Mask") (roundrect_rratio 0.25) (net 6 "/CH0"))
  (pad "2" smd roundrect (at -2.8625 1.625 270) (size 1.475 0.4) (layers "B.Cu" "B.Paste" "B.Mask") (roundrect_rratio 0.25) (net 7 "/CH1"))
  (pad "3" smd roundrect (at -2.8625 0.975 270) (size 1.475 0.4) (layers "B.Cu" "B.Paste" "B.Mask") (roundrect_rratio 0.25) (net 2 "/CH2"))
  (pad "4" smd roundrect (at -2.8625 0.325 270) (size 1.475 0.4) (layers "B.Cu" "B.Paste" "B.Mask") (roundrect_rratio 0.25) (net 5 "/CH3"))
  (pad "5" smd roundrect (at -2.8625 -0.325 270) (size 1.475 0.4) (layers "B.Cu" "B.Paste" "B.Mask") (roundrect_rratio 0.25) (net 4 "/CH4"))
  (pad "6" smd roundrect (at -2.8625 -0.975 270) (size 1.475 0.4) (layers "B.Cu" "B.Paste" "B.Mask") (roundrect_rratio 0.25) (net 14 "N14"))
  (pad "7" smd roundrect (at -2.8625 -1.625 270) (size 1.475 0.4) (layers "B.Cu" "B.Paste" "B.Mask") (roundrect_rratio 0.25) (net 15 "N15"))
  (pad "8" smd roundrect (at -2.8625 -2.275 270) (size 1.475 0.4) (layers "B.Cu" "B.Paste" "B.Mask") (roundrect_rratio 0.25) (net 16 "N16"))
  (pad "9" smd roundrect (at 2.8625 -2.275 270) (size 1.475 0.4) (layers "B.Cu" "B.Paste" "B.Mask") (roundrect_rratio 0.25) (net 3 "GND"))
  (pad "10" smd roundrect (at 2.8625 -1.625 270) (size 1.475 0.4) (layers "B.Cu" "B.Paste" "B.Mask") (roundrect_rratio 0.25) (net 1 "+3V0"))
  (pad "11" smd roundrect (at 2.8625 -0.975 270) (size 1.475 0.4) (layers "B.Cu" "B.Paste" "B.Mask") (roundrect_rratio 0.25) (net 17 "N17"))
  (pad "12" smd roundrect (at 2.8625 -0.325 270) (size 1.475 0.4) (layers "B.Cu" "B.Paste" "B.Mask") (roundrect_rratio 0.25) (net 9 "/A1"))
  (pad "13" smd roundrect (at 2.8625 0.325 270) (size 1.475 0.4) (layers "B.Cu" "B.Paste" "B.Mask") (roundrect_rratio 0.25) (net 10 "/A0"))
  (pad "14" smd roundrect (at 2.8625 0.975 270) (size 1.475 0.4) (layers "B.Cu" "B.Paste" "B.Mask") (roundrect_rratio 0.25) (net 12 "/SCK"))
  (pad "15" smd roundrect (at 2.8625 1.625 270) (size 1.475 0.4) (layers "B.Cu" "B.Paste" "B.Mask") (roundrect_rratio 0.25) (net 11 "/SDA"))
  (pad "16" smd roundrect (at 2.8625 2.275 270) (size 1.475 0.4) (layers "B.Cu" "B.Paste" "B.Mask") (roundrect_rratio 0.25) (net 8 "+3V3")))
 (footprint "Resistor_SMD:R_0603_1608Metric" (layer "B.Cu") (at 113.25 126.2625)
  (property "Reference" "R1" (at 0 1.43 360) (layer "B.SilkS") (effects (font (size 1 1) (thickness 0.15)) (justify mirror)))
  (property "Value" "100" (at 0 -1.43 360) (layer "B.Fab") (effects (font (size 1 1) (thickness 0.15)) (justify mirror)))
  (pad "1" smd roundrect (at -0.825 0) (size 0.8 0.95) (layers "B.Cu" "B.Paste" "B.Mask") (roundrect_rratio 0.25) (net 8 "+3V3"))
  (pad "2" smd roundrect (at 0.825 0) (size 0.8 0.95) (layers "B.Cu" "B.Paste" "B.Mask") (roundrect_rratio 0.25) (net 1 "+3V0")))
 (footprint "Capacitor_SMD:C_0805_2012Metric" (layer "B.Cu") (at 103.2 121.6 90)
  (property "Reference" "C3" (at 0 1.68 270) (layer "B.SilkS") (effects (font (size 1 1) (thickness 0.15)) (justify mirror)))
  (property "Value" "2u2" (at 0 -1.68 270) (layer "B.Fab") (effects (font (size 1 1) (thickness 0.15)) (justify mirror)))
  (pad "1" smd roundrect (at -0.95 0 90) (size 1 1.45) (layers "B.Cu" "B.Paste" "B.Mask") (roundrect_rratio 0.25) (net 8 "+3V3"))
  (pad "2" smd roundrect (at 0.95 0 90) (size 1 1.45) (layers "B.Cu" "B.Paste" "B.Mask") (roundrect_rratio 0.25) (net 3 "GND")))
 (gr_line (start 88 139) (end 188 139) (stroke (width 0.05) (type default)) (layer "Edge.Cuts"))
 (gr_line (start 88 61) (end 88 139) (stroke (width 0.05) (type default)) (layer "Edge.Cuts"))
 (gr_line (start 188 139) (end 188 61) (stroke (width 0.05) (type default)) (layer "Edge.Cuts"))
 (gr_line (start 188 61) (end 88 61) (stroke (width 0.05) (type default)) (layer "Edge.Cuts"))
 (segment (start 112.2 120.4625) (end 112.2 118.8375) (width 0.2) (layer "B.Cu") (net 1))
 (segment (start 112.375 120.6375) (end 112.2 120.4625) (width 0.2) (layer "B.Cu") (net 1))
 (segment (start 112.2 118.8375) (end 112.375 118.6625) (width 0.2) (layer "B.Cu") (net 1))
 (segment (start 110.225 122.2625) (end 110.225 121.175) (width 0.2) (layer "B.Cu") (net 1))
 (segment (start 110.225 121.175) (end 110.9375 120.4625) (width 0.2) (layer "B.Cu") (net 1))
 (segment (start 110.9375 120.4625) (end 112.2 120.4625) (width 0.2) (layer "B.Cu") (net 1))
 (segment (start 112.375 122.525) (end 112.375 120.6375) (width 0.2) (layer "B.Cu") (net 1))
 (segment (start 110.6 126.8125) (end 110.6 129.3425) (width 0.5) (layer "B.Cu") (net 3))
 (segment (start 110.875 122.2625) (end 110.875 126.5375) (width 0.3) (layer "B.Cu") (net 3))
 (segment (start 110.875 126.5375) (end 110.6 126.8125) (width 0.3) (layer "B.Cu") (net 3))
 (segment (start 105 122.575) (end 102.125 122.575) (width 0.5) (layer "B.Cu") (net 8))
 (segment (start 102.125 122.575) (end 100.825 123.875) (width 0.5) (layer "B.Cu") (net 8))
 (segment (start 106.0125 122.575) (end 105 122.575) (width 0.3) (layer "B.Cu") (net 8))
 (segment (start 100.825 123.875) (end 100.825 124.1) (width 0.5) (layer "B.Cu") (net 8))
 (segment (start 106.325 122.2625) (end 106.0125 122.575) (width 0.3) (layer "B.Cu") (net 8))
 (segment (start 108 126.8125) (end 108 129.3425) (width 0.5) (layer "B.Cu") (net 8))
 (segment (start 108.7 125.1) (end 109.3 125.7) (width 0.2) (layer "F.Cu") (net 10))
 (segment (start 109.3 125.7) (end 109.3 128.1) (width 0.2) (layer "F.Cu") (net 10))
 (via (at 109.3 128.1) (size 0.6) (drill 0.3) (layers "F.Cu" "B.Cu") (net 10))
 (via (at 108.7 125.1) (size 0.6) (drill 0.3) (layers "F.Cu" "B.Cu") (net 10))
 (segment (start 108.275 122.2625) (end 108.275 124.675) (width 0.2) (layer "B.Cu") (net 10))
 (segment (start 109.3 128.1) (end 109.3 129.3425) (width 0.2) (layer "B.Cu") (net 10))
 (segment (start 108.275 124.675) (end 108.7 125.1) (width 0.2) (layer "B.Cu") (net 10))
 (segment (start 109.3 124.8) (end 108.925 124.425) (width 0.2) (layer "B.Cu") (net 9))
 (segment (start 108.925 124.425) (end 108.925 122.2625) (width 0.2) (layer "B.Cu") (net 9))
 (segment (start 109.3 126.8125) (end 109.3 124.8) (width 0.2) (layer "B.Cu") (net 9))
 (segment (start 105.2 125.1) (end 100.825 125.1) (width 0.2) (layer "B.Cu") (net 11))
 (segment (start 106.975 123.325) (end 105.2 125.1) (width 0.2) (layer "B.Cu") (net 11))
 (segment (start 106.975 122.2625) (end 106.975 123.325) (width 0.2) (layer "B.Cu") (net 11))
 (segment (start 107.625 123.875) (end 105.4 126.1) (width 0.2) (layer "B.Cu") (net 12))
 (segment (start 105.4 126.1) (end 100.825 126.1) (width 0.2) (layer "B.Cu") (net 12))
 (segment (start 107.625 122.2625) (end 107.625 123.875) (width 0.2) (layer "B.Cu") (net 12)))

